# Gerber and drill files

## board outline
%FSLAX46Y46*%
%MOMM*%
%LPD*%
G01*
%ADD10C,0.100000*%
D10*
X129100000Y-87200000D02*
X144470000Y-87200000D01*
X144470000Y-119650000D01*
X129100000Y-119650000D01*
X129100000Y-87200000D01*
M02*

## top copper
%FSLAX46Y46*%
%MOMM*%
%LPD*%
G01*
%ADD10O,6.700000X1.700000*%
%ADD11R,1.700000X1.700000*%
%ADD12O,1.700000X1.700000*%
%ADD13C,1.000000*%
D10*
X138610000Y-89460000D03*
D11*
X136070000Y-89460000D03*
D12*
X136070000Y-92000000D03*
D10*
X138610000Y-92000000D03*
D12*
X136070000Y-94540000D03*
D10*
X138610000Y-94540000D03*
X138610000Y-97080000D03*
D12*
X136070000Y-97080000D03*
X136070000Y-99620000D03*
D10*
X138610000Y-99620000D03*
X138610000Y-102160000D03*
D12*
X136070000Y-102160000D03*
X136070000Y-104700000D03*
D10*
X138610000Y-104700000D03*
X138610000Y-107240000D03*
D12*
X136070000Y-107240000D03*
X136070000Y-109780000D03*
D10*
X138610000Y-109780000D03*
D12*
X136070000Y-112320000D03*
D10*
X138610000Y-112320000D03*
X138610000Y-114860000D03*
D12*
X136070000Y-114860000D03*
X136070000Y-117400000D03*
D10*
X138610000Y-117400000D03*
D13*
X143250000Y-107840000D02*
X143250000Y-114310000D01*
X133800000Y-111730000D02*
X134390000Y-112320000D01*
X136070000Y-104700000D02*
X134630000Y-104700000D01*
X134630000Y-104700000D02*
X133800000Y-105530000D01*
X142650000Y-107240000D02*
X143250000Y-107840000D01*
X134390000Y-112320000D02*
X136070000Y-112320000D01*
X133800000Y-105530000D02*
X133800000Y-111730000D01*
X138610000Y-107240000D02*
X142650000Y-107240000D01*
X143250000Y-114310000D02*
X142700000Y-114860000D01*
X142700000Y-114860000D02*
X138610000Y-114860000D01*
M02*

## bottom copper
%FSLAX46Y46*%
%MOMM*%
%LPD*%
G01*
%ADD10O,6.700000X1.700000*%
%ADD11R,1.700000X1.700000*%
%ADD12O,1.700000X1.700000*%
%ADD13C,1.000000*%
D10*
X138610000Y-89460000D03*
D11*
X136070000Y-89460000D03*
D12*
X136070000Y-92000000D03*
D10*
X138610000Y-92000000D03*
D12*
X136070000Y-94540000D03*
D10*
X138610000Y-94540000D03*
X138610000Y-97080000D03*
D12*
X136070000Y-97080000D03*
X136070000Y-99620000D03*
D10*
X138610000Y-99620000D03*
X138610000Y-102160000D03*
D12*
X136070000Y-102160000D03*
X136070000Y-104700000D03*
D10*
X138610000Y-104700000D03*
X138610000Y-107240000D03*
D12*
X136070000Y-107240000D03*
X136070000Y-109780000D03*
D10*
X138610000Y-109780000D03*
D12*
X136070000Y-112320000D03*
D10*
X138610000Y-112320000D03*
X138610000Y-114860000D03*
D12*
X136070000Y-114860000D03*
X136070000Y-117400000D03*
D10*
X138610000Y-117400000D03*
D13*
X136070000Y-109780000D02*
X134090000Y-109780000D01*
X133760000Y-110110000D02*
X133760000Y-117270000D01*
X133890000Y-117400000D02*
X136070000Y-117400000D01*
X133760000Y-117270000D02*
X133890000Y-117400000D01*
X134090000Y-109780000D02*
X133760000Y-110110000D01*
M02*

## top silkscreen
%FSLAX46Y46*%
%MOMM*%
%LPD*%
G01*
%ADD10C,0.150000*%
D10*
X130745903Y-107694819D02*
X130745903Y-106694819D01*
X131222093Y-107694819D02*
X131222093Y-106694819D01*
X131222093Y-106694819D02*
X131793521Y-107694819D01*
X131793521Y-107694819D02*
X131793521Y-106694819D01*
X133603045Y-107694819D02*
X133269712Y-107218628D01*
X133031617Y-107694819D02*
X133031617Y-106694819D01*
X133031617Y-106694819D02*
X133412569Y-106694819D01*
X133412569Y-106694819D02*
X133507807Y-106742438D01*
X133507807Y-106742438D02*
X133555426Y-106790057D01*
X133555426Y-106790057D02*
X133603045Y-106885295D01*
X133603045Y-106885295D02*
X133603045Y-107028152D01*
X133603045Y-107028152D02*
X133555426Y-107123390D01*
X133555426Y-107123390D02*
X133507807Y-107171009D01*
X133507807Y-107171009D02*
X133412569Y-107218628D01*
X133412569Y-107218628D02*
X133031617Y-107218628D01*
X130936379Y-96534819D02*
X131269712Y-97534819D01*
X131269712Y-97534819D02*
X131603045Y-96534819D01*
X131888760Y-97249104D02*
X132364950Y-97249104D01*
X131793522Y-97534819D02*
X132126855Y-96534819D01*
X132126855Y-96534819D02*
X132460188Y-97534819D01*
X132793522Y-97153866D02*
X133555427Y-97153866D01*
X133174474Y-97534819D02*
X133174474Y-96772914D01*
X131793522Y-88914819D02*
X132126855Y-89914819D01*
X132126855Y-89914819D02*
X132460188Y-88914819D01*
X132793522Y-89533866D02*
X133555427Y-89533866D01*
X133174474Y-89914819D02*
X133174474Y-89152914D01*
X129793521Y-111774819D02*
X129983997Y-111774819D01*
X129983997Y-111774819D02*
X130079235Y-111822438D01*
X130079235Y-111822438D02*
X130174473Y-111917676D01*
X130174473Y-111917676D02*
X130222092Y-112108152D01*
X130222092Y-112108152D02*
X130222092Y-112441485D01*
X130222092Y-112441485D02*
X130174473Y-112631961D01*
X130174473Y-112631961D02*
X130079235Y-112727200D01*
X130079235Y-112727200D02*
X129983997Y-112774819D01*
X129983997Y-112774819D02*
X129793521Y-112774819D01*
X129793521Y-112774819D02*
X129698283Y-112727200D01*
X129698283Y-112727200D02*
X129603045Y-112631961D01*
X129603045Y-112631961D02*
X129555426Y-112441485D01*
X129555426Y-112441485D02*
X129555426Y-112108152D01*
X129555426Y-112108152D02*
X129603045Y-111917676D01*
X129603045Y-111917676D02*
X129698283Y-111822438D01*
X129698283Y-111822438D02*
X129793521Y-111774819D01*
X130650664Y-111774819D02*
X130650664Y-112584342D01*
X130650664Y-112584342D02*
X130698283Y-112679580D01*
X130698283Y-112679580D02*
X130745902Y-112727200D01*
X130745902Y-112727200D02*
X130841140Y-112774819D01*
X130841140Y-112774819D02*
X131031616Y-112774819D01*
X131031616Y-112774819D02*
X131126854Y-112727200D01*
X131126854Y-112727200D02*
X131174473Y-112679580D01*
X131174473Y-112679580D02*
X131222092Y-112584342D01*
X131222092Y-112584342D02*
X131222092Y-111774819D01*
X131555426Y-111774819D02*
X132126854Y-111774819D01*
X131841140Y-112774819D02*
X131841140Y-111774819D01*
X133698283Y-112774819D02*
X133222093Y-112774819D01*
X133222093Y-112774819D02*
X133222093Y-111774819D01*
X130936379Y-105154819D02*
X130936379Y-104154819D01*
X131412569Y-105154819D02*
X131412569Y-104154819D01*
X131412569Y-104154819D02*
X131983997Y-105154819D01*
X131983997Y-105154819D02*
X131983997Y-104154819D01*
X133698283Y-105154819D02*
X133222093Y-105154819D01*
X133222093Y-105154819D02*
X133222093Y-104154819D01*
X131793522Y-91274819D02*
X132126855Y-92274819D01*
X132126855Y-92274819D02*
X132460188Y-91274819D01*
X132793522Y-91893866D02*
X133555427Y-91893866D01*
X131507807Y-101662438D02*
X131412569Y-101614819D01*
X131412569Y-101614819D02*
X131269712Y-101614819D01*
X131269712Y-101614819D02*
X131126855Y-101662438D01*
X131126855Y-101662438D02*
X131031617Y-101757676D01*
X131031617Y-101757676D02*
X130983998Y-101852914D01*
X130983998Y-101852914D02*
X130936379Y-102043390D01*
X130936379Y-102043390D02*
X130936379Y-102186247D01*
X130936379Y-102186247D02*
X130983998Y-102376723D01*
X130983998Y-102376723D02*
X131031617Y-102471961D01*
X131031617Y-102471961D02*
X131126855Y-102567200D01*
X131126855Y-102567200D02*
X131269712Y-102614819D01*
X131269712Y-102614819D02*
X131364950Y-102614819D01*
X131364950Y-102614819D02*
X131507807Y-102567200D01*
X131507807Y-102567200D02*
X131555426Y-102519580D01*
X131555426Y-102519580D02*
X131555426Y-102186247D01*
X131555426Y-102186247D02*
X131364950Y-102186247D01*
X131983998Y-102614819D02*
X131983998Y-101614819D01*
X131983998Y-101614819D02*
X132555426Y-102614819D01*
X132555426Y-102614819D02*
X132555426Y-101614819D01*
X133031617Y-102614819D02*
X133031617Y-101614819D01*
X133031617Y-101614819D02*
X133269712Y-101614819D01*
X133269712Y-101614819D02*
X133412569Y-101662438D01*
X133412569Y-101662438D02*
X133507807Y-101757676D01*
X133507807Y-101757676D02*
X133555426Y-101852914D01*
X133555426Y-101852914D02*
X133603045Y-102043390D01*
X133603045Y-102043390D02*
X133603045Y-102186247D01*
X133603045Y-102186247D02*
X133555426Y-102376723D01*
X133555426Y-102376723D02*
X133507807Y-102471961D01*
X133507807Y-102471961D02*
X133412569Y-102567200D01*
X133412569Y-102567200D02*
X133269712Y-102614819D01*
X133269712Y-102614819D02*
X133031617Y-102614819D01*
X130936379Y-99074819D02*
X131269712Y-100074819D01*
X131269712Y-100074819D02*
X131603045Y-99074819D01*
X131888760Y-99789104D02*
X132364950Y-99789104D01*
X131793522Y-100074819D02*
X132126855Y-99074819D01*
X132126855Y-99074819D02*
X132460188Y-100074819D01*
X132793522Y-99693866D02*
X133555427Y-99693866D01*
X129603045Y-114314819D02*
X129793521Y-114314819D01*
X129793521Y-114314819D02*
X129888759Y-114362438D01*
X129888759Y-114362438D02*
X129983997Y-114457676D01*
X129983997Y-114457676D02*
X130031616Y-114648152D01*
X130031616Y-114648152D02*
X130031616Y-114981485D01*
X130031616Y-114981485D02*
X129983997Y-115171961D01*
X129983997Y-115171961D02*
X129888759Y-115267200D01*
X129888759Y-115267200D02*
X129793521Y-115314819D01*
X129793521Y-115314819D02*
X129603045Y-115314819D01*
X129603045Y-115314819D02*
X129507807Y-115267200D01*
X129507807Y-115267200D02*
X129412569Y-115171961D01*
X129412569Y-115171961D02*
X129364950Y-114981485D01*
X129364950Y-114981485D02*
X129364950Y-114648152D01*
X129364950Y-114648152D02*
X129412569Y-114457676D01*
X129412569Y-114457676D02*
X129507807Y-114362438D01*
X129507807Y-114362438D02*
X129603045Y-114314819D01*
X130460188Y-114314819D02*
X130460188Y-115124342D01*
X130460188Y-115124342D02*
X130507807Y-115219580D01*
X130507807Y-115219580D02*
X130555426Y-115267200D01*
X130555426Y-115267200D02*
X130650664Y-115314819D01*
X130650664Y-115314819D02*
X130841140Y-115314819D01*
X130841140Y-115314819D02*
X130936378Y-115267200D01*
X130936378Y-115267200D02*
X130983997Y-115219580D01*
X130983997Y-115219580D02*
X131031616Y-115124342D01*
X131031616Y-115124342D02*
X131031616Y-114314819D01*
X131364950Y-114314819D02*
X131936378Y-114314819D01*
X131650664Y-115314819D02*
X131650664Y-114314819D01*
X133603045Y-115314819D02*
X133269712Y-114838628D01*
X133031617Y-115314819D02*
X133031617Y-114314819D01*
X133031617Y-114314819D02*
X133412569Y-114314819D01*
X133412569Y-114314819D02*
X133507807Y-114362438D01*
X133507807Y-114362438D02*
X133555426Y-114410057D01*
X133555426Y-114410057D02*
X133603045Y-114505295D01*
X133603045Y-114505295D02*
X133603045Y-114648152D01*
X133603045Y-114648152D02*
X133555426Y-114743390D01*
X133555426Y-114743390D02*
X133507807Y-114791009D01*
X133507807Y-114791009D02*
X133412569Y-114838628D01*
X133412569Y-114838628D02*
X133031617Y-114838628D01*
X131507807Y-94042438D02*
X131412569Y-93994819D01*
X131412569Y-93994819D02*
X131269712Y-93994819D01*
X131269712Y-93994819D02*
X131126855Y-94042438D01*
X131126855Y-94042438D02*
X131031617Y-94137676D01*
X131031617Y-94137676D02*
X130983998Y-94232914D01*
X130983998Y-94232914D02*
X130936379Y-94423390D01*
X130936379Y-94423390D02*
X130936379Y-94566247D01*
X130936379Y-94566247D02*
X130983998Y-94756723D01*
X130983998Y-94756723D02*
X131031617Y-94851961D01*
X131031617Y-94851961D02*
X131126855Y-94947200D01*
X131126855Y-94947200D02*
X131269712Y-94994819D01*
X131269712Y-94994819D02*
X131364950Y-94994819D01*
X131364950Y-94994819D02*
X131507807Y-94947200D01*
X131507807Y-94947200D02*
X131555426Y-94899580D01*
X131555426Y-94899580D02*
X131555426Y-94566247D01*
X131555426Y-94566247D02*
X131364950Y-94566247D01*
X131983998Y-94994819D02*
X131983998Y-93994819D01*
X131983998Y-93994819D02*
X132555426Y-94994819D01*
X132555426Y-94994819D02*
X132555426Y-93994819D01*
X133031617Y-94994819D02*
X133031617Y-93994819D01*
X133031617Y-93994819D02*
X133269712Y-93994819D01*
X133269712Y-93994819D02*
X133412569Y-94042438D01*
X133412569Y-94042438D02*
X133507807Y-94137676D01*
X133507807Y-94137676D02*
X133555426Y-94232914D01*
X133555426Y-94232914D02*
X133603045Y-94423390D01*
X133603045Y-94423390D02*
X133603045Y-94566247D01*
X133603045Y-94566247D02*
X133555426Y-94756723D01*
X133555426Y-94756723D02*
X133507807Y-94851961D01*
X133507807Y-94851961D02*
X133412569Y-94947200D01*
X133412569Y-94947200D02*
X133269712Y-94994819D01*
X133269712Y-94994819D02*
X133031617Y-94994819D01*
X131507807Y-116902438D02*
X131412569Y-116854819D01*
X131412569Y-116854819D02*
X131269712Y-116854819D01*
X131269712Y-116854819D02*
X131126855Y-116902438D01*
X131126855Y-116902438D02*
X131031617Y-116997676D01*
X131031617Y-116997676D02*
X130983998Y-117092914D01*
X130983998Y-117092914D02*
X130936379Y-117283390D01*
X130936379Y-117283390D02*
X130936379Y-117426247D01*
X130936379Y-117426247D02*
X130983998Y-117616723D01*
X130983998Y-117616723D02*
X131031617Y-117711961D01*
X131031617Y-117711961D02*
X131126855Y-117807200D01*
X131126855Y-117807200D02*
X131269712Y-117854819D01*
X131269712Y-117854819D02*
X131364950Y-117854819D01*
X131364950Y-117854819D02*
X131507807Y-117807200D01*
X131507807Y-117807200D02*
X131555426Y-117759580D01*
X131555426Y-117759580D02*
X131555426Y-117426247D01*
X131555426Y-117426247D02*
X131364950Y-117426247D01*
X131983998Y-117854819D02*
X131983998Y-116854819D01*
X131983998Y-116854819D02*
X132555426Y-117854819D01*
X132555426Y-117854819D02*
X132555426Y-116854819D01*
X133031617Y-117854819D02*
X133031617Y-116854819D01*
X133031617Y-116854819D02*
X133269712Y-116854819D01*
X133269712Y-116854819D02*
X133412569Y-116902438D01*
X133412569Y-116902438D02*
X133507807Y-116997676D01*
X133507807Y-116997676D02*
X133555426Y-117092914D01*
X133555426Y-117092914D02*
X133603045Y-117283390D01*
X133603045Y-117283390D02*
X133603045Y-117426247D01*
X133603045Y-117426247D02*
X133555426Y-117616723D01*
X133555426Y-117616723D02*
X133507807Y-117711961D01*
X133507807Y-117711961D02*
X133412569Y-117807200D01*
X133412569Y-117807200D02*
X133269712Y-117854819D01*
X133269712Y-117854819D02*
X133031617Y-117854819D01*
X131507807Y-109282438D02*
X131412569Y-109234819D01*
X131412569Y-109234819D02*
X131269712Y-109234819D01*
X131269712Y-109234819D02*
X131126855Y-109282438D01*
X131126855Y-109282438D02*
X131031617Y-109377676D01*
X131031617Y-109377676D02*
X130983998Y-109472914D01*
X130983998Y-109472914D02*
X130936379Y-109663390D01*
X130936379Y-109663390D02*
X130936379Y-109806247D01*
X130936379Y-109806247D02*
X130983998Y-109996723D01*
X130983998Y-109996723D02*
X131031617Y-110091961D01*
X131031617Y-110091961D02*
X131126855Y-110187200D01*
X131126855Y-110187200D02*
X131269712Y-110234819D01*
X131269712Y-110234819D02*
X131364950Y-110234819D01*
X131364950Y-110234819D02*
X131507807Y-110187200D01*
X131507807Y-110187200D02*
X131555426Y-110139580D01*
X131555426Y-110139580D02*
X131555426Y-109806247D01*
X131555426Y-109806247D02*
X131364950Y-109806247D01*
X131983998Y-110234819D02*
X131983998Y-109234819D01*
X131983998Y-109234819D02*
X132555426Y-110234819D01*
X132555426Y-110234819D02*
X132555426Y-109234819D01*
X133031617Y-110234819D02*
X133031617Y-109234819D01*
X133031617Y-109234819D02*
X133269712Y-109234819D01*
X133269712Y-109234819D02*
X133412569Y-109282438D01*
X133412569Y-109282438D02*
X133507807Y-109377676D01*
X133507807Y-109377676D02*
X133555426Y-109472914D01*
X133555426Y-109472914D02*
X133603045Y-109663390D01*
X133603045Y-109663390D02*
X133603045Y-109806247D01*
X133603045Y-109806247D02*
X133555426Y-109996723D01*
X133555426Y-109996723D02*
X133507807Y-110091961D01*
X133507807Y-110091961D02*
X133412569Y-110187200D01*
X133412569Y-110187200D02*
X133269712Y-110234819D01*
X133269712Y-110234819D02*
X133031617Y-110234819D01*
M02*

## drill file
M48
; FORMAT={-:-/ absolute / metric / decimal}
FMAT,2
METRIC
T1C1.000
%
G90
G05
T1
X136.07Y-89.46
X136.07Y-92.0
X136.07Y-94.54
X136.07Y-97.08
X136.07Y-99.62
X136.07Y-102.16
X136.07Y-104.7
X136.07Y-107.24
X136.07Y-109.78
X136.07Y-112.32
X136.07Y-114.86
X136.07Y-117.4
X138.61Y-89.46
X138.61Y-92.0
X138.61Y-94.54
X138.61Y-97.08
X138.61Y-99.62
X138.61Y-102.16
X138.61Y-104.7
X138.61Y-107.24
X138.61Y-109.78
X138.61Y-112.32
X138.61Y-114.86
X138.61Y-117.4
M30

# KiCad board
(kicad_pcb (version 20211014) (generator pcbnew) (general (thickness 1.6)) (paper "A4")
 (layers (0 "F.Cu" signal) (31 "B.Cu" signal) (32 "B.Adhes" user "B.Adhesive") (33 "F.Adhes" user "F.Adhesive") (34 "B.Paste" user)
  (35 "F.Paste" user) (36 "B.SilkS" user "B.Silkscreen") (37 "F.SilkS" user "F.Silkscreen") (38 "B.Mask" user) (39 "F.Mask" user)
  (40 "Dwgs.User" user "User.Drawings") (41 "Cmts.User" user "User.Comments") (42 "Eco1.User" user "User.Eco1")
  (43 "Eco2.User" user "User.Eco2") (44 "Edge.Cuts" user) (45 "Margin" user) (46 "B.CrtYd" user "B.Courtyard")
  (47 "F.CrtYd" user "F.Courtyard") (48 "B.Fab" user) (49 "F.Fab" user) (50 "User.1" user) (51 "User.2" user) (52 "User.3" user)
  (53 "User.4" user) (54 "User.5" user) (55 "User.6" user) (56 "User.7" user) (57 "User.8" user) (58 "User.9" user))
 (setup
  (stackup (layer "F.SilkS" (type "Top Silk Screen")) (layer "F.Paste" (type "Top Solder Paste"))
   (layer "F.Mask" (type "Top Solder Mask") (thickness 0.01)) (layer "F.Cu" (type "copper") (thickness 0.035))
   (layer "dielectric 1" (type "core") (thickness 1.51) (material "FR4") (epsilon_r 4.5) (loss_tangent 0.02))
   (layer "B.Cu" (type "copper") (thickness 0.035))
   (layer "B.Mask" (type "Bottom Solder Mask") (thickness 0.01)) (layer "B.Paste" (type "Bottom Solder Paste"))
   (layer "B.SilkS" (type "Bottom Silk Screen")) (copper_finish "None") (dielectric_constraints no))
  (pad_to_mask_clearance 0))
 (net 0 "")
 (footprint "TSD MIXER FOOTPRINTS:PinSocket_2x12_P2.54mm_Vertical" (layer "F.Cu") (at 136.07 89.46)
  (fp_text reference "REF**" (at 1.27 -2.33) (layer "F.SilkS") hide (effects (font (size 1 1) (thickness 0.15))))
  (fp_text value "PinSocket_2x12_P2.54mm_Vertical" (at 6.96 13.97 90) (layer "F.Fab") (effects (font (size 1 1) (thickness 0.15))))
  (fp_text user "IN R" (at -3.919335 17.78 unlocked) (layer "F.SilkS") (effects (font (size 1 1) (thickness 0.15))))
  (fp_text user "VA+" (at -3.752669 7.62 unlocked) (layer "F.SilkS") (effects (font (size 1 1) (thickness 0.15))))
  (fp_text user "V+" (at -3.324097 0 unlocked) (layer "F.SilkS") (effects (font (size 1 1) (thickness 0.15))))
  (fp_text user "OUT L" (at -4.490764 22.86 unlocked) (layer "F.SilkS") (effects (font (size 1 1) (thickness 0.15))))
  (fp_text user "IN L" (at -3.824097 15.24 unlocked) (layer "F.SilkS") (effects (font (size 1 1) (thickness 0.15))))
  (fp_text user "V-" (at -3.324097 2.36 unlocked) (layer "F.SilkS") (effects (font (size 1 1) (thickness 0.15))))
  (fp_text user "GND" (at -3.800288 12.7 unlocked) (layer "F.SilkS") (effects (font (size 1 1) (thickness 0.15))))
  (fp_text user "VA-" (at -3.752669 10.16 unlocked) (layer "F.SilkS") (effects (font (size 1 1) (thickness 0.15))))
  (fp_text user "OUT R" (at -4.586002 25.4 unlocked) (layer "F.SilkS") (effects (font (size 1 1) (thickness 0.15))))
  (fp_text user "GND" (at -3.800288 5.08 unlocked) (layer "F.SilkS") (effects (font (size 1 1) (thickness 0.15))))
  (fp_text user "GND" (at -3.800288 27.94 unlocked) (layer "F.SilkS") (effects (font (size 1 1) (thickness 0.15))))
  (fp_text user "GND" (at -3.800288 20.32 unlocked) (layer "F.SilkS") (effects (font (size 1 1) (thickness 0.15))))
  (pad "1" thru_hole oval (at 2.54 0) (size 6.7 1.7) (drill 1) (layers *.Cu *.Mask))
  (pad "1" thru_hole rect (at 0 0) (size 1.7 1.7) (drill 1) (layers *.Cu *.Mask))
  (pad "2" thru_hole oval (at 0 2.54) (size 1.7 1.7) (drill 1) (layers *.Cu *.Mask))
  (pad "2" thru_hole oval (at 2.54 2.54) (size 6.7 1.7) (drill 1) (layers *.Cu *.Mask))
  (pad "3" thru_hole oval (at 0 5.08) (size 1.7 1.7) (drill 1) (layers *.Cu *.Mask))
  (pad "3" thru_hole oval (at 2.54 5.08) (size 6.7 1.7) (drill 1) (layers *.Cu *.Mask))
  (pad "4" thru_hole oval (at 2.54 7.62) (size 6.7 1.7) (drill 1) (layers *.Cu *.Mask))
  (pad "4" thru_hole oval (at 0 7.62) (size 1.7 1.7) (drill 1) (layers *.Cu *.Mask))
  (pad "5" thru_hole oval (at 0 10.16) (size 1.7 1.7) (drill 1) (layers *.Cu *.Mask))
  (pad "5" thru_hole oval (at 2.54 10.16) (size 6.7 1.7) (drill 1) (layers *.Cu *.Mask))
  (pad "6" thru_hole oval (at 2.54 12.7) (size 6.7 1.7) (drill 1) (layers *.Cu *.Mask))
  (pad "6" thru_hole oval (at 0 12.7) (size 1.7 1.7) (drill 1) (layers *.Cu *.Mask))
  (pad "7" thru_hole oval (at 0 15.24) (size 1.7 1.7) (drill 1) (layers *.Cu *.Mask))
  (pad "7" thru_hole oval (at 2.54 15.24) (size 6.7 1.7) (drill 1) (layers *.Cu *.Mask))
  (pad "8" thru_hole oval (at 2.54 17.78) (size 6.7 1.7) (drill 1) (layers *.Cu *.Mask))
  (pad "8" thru_hole oval (at 0 17.78) (size 1.7 1.7) (drill 1) (layers *.Cu *.Mask))
  (pad "9" thru_hole oval (at 0 20.32) (size 1.7 1.7) (drill 1) (layers *.Cu *.Mask))
  (pad "9" thru_hole oval (at 2.54 20.32) (size 6.7 1.7) (drill 1) (layers *.Cu *.Mask))
  (pad "10" thru_hole oval (at 0 22.86) (size 1.7 1.7) (drill 1) (layers *.Cu *.Mask))
  (pad "10" thru_hole oval (at 2.54 22.86) (size 6.7 1.7) (drill 1) (layers *.Cu *.Mask))
  (pad "11" thru_hole oval (at 2.54 25.4) (size 6.7 1.7) (drill 1) (layers *.Cu *.Mask))
  (pad "11" thru_hole oval (at 0 25.4) (size 1.7 1.7) (drill 1) (layers *.Cu *.Mask))
  (pad "12" thru_hole oval (at 0 27.94) (size 1.7 1.7) (drill 1) (layers *.Cu *.Mask))
  (pad "12" thru_hole oval (at 2.54 27.94) (size 6.7 1.7) (drill 1) (layers *.Cu *.Mask)))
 (gr_rect (start 144.47 119.65) (end 129.1 87.2) (layer "Edge.Cuts") (width 0.1) (fill none))
 (segment (start 143.25 107.84) (end 143.25 114.31) (width 1) (layer "F.Cu") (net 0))
 (segment (start 133.8 111.73) (end 134.39 112.32) (width 1) (layer "F.Cu") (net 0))
 (segment (start 136.07 104.7) (end 134.63 104.7) (width 1) (layer "F.Cu") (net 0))
 (segment (start 134.63 104.7) (end 133.8 105.53) (width 1) (layer "F.Cu") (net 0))
 (segment (start 142.65 107.24) (end 143.25 107.84) (width 1) (layer "F.Cu") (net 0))
 (segment (start 134.39 112.32) (end 136.07 112.32) (width 1) (layer "F.Cu") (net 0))
 (segment (start 133.8 105.53) (end 133.8 111.73) (width 1) (layer "F.Cu") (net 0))
 (segment (start 138.61 107.24) (end 142.65 107.24) (width 1) (layer "F.Cu") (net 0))
 (segment (start 143.25 114.31) (end 142.7 114.86) (width 1) (layer "F.Cu") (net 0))
 (segment (start 142.7 114.86) (end 138.61 114.86) (width 1) (layer "F.Cu") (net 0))
 (segment (start 136.07 109.78) (end 134.09 109.78) (width 1) (layer "B.Cu") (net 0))
 (segment (start 133.76 110.11) (end 133.76 117.27) (width 1) (layer "B.Cu") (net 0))
 (segment (start 133.89 117.4) (end 136.07 117.4) (width 1) (layer "B.Cu") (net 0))
 (segment (start 133.76 117.27) (end 133.89 117.4) (width 1) (layer "B.Cu") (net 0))
 (segment (start 134.09 109.78) (end 133.76 110.11) (width 1) (layer "B.Cu") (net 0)))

